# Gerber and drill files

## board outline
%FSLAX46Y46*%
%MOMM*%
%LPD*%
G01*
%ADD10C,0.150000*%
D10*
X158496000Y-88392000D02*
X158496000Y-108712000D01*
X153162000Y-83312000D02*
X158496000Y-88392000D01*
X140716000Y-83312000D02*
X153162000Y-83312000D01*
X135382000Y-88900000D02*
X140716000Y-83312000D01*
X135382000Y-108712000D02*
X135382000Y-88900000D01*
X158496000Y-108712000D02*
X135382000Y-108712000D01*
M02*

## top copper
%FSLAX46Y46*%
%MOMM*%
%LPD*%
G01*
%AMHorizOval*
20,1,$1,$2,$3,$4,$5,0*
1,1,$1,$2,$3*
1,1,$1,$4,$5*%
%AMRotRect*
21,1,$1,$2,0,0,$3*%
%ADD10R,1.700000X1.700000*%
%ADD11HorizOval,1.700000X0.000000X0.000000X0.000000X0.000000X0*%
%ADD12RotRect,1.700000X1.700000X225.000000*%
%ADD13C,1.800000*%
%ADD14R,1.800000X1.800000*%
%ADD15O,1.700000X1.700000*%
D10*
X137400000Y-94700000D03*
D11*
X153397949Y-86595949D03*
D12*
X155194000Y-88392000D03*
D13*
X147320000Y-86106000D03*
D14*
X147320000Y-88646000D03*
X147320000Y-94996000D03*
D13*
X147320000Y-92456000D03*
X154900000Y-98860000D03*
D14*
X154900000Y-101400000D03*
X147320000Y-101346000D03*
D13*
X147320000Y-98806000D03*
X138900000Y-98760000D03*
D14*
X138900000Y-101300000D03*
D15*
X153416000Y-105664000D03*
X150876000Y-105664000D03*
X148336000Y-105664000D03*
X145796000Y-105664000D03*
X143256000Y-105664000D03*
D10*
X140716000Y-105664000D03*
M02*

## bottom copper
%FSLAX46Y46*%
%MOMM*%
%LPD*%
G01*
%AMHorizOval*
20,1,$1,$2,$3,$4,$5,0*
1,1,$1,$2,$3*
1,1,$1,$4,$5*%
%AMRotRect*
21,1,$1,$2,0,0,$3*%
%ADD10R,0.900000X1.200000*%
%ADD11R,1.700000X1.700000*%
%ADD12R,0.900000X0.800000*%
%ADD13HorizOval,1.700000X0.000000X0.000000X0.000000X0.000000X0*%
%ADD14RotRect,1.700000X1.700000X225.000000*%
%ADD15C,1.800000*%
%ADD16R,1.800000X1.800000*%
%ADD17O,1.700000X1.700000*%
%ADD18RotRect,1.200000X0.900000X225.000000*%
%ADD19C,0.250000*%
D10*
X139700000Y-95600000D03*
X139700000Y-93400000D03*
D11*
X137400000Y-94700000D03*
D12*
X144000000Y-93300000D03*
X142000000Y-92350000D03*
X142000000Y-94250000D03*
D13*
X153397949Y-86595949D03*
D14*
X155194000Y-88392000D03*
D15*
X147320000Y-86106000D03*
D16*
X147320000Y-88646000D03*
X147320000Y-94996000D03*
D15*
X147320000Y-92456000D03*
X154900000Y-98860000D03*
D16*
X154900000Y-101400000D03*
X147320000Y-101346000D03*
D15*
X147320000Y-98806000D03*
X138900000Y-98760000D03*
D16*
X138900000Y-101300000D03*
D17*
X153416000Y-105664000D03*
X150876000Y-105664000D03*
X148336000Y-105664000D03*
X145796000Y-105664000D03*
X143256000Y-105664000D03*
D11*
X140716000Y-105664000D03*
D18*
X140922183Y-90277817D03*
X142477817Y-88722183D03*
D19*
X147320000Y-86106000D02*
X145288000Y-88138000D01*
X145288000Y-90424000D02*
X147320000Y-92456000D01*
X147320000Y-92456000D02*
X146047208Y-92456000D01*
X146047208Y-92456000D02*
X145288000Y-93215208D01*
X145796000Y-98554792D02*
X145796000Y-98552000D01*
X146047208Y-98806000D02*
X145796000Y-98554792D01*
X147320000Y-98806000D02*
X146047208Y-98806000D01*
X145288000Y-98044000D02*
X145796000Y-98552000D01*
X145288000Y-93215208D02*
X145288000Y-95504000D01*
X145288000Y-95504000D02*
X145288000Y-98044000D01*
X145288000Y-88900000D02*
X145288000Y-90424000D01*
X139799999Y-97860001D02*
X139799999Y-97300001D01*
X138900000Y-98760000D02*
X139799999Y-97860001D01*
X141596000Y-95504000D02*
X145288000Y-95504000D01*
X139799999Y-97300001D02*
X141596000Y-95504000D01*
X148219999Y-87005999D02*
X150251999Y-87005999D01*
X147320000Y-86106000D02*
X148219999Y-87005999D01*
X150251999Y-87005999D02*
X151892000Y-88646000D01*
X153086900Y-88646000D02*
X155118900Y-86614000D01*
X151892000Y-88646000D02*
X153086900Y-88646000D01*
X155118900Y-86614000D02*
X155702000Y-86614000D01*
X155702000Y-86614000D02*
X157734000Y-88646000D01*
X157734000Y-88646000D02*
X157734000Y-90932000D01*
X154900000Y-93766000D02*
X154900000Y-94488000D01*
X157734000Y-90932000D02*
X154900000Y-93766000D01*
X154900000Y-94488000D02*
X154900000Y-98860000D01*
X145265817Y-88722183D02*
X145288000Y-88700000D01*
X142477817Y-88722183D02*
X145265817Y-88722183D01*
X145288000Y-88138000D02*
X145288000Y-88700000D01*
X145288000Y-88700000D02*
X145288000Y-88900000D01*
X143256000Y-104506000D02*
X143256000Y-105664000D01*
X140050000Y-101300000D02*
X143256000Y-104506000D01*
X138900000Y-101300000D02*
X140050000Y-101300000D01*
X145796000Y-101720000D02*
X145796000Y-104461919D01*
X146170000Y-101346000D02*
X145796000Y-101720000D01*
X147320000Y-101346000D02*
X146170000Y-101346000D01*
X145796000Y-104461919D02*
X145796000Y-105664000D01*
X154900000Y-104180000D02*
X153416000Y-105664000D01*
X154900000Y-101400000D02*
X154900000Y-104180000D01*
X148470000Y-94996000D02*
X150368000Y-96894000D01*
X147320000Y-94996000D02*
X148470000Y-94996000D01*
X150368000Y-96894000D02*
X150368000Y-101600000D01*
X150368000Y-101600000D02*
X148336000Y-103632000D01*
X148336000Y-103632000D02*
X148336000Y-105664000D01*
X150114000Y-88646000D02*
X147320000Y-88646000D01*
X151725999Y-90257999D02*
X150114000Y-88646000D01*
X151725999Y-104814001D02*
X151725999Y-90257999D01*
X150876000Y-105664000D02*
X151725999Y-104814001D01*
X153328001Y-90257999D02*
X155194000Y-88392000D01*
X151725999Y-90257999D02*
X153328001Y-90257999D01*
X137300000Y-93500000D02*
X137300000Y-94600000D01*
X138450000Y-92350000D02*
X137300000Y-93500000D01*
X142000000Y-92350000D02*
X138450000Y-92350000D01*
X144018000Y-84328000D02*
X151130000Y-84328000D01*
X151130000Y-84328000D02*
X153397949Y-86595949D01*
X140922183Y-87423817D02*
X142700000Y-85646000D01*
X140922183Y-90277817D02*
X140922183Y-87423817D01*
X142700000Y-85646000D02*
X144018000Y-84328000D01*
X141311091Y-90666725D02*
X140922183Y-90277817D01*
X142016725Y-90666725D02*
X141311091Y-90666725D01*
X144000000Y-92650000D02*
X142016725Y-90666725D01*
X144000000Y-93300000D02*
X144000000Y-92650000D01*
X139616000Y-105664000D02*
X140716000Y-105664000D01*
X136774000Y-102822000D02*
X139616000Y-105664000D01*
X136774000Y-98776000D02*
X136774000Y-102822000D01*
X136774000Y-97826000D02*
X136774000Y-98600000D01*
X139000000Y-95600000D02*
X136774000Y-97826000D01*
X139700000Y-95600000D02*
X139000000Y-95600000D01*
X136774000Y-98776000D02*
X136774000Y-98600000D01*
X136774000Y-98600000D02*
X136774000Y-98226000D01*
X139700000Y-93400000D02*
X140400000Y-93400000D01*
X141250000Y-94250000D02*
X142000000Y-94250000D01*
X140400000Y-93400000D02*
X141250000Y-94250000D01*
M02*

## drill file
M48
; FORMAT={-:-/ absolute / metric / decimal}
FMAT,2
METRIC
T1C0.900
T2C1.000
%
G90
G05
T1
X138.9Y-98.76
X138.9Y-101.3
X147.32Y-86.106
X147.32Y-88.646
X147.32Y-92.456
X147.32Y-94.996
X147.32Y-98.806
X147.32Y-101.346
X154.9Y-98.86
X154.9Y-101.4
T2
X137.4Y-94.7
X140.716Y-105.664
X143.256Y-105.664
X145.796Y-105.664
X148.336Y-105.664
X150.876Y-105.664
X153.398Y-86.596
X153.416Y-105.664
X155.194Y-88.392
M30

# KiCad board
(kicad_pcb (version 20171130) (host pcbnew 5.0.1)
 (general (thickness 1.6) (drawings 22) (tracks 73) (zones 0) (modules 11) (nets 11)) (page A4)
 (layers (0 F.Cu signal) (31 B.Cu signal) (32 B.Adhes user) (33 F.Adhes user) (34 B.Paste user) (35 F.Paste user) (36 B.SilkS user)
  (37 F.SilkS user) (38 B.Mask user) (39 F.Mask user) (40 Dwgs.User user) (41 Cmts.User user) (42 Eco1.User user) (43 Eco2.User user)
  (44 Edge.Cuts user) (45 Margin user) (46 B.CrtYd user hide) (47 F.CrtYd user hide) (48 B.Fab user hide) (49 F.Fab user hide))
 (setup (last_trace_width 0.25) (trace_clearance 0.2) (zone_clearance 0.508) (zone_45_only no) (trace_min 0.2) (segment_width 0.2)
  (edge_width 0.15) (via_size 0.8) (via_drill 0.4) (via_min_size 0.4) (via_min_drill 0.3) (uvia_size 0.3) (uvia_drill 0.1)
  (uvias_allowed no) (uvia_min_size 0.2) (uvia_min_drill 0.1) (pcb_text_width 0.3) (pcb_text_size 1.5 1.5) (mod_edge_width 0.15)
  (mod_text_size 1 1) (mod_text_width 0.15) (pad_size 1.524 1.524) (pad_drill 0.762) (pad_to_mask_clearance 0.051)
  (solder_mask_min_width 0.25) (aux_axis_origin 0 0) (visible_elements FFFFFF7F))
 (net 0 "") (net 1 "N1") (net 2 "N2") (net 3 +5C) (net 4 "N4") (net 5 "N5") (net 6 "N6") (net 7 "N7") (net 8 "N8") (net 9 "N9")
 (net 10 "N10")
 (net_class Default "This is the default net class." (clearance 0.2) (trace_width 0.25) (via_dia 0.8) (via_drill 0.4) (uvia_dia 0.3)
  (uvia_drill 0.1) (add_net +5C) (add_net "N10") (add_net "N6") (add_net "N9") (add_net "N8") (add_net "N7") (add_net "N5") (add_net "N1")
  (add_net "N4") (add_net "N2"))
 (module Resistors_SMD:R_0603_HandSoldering (layer B.Cu) (at 139.7 94.5 270)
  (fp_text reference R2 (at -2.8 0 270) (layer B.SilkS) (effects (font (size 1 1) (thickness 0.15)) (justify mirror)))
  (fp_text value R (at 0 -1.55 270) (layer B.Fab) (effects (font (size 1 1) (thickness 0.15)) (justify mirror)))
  (pad 2 smd rect (at 1.1 0 270) (size 1.2 0.9) (layers B.Cu B.Paste B.Mask) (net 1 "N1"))
  (pad 1 smd rect (at -1.1 0 270) (size 1.2 0.9) (layers B.Cu B.Paste B.Mask) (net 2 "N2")))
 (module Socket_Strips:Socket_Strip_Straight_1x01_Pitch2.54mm (layer F.Cu) (at 137.4 94.7)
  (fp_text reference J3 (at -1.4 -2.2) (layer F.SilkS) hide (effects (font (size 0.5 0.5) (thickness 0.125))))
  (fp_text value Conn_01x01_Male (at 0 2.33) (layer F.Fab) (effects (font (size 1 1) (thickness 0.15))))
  (pad 1 thru_hole rect (at 0 0) (size 1.7 1.7) (drill 1) (layers *.Cu *.Mask) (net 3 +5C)))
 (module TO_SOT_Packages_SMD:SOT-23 (layer B.Cu) (at 143 93.3)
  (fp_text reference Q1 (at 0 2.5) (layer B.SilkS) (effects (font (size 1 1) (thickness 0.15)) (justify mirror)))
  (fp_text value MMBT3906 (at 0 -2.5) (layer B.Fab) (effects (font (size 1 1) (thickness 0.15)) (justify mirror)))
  (pad 3 smd rect (at 1 0) (size 0.9 0.8) (layers B.Cu B.Paste B.Mask) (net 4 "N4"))
  (pad 2 smd rect (at -1 -0.95) (size 0.9 0.8) (layers B.Cu B.Paste B.Mask) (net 3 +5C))
  (pad 1 smd rect (at -1 0.95) (size 0.9 0.8) (layers B.Cu B.Paste B.Mask) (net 2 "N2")))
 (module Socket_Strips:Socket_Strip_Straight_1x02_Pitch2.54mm (layer F.Cu) (at 155.194 88.392 225)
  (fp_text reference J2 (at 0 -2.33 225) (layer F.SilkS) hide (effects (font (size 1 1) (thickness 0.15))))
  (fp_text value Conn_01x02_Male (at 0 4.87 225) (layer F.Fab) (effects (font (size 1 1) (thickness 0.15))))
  (pad 2 thru_hole oval (at 0 2.54 225) (size 1.7 1.7) (drill 1) (layers *.Cu *.Mask) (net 4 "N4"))
  (pad 1 thru_hole rect (at 0 0 225) (size 1.7 1.7) (drill 1) (layers *.Cu *.Mask) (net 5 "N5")))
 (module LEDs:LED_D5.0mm (layer F.Cu) (at 147.32 88.646 90)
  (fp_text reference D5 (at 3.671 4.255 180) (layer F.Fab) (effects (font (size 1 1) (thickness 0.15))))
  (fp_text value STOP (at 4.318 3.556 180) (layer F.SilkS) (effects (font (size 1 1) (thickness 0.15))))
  (pad 2 thru_hole circle (at 2.54 0 90) (size 1.8 1.8) (drill 0.9) (layers *.Cu *.Mask) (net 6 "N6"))
  (pad 1 thru_hole rect (at 0 0 90) (size 1.8 1.8) (drill 0.9) (layers *.Cu *.Mask) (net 5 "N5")))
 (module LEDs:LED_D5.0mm (layer F.Cu) (at 147.32 94.996 90)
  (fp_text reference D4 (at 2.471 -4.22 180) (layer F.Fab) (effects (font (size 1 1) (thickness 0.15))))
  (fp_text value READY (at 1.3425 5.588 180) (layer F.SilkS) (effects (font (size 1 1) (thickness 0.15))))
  (pad 1 thru_hole rect (at 0 0 90) (size 1.8 1.8) (drill 0.9) (layers *.Cu *.Mask) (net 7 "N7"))
  (pad 2 thru_hole circle (at 2.54 0 90) (size 1.8 1.8) (drill 0.9) (layers *.Cu *.Mask) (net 6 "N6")))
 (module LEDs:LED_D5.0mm (layer F.Cu) (at 154.9 101.4 90)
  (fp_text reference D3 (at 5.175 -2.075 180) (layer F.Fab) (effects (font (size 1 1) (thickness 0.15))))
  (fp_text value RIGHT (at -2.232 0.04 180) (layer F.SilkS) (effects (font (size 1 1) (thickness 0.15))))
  (pad 2 thru_hole circle (at 2.54 0 90) (size 1.8 1.8) (drill 0.9) (layers *.Cu *.Mask) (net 6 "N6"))
  (pad 1 thru_hole rect (at 0 0 90) (size 1.8 1.8) (drill 0.9) (layers *.Cu *.Mask) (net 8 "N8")))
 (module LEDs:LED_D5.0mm (layer F.Cu) (at 147.32 101.346 90)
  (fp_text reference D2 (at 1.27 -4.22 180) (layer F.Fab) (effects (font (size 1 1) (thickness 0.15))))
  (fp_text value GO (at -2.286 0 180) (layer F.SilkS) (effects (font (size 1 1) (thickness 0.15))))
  (pad 1 thru_hole rect (at 0 0 90) (size 1.8 1.8) (drill 0.9) (layers *.Cu *.Mask) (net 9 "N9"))
  (pad 2 thru_hole circle (at 2.54 0 90) (size 1.8 1.8) (drill 0.9) (layers *.Cu *.Mask) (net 6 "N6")))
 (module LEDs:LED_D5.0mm (layer F.Cu) (at 138.9 101.3 90)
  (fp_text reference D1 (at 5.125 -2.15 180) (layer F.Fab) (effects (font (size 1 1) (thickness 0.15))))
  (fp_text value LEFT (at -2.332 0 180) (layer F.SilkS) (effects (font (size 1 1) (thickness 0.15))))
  (pad 2 thru_hole circle (at 2.54 0 90) (size 1.8 1.8) (drill 0.9) (layers *.Cu *.Mask) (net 6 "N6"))
  (pad 1 thru_hole rect (at 0 0 90) (size 1.8 1.8) (drill 0.9) (layers *.Cu *.Mask) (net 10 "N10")))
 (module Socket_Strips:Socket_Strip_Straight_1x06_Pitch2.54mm (layer F.Cu) (at 140.716 105.664 90)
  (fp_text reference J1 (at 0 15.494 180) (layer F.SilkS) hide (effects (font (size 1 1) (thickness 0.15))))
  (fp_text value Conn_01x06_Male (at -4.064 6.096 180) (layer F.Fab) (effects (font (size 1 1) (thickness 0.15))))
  (pad 6 thru_hole oval (at 0 12.7 90) (size 1.7 1.7) (drill 1) (layers *.Cu *.Mask) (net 8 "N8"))
  (pad 5 thru_hole oval (at 0 10.16 90) (size 1.7 1.7) (drill 1) (layers *.Cu *.Mask) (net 5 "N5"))
  (pad 4 thru_hole oval (at 0 7.62 90) (size 1.7 1.7) (drill 1) (layers *.Cu *.Mask) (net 7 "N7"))
  (pad 3 thru_hole oval (at 0 5.08 90) (size 1.7 1.7) (drill 1) (layers *.Cu *.Mask) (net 9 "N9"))
  (pad 2 thru_hole oval (at 0 2.54 90) (size 1.7 1.7) (drill 1) (layers *.Cu *.Mask) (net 10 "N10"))
  (pad 1 thru_hole rect (at 0 0 90) (size 1.7 1.7) (drill 1) (layers *.Cu *.Mask) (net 1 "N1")))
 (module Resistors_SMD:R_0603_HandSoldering (layer B.Cu) (at 141.7 89.5 225)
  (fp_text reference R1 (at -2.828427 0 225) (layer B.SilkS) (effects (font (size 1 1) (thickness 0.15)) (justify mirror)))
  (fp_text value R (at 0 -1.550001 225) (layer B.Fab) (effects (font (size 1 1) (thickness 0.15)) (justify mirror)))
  (pad 2 smd rect (at 1.099999 0 225) (size 1.2 0.9) (layers B.Cu B.Paste B.Mask) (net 4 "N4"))
  (pad 1 smd rect (at -1.099999 0 225) (size 1.2 0.9) (layers B.Cu B.Paste B.Mask) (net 6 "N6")))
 (gr_line (start 158.496 88.392) (end 158.496 108.712) (layer Edge.Cuts) (width 0.15))
 (gr_line (start 153.162 83.312) (end 158.496 88.392) (layer Edge.Cuts) (width 0.15))
 (gr_line (start 140.716 83.312) (end 153.162 83.312) (layer Edge.Cuts) (width 0.15))
 (gr_line (start 135.382 88.9) (end 140.716 83.312) (layer Edge.Cuts) (width 0.15))
 (gr_line (start 135.382 108.712) (end 135.382 88.9) (layer Edge.Cuts) (width 0.15))
 (gr_line (start 158.496 108.712) (end 135.382 108.712) (layer Edge.Cuts) (width 0.15))
 (segment (start 147.32 86.106) (end 145.288 88.138) (width 0.25) (layer B.Cu) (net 6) (status 10))
 (segment (start 145.288 90.424) (end 147.32 92.456) (width 0.25) (layer B.Cu) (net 6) (status 20))
 (segment (start 147.32 92.456) (end 146.047208 92.456) (width 0.25) (layer B.Cu) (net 6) (status 10))
 (segment (start 146.047208 92.456) (end 145.288 93.215208) (width 0.25) (layer B.Cu) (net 6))
 (segment (start 145.796 98.554792) (end 145.796 98.552) (width 0.25) (layer B.Cu) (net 6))
 (segment (start 146.047208 98.806) (end 145.796 98.554792) (width 0.25) (layer B.Cu) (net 6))
 (segment (start 147.32 98.806) (end 146.047208 98.806) (width 0.25) (layer B.Cu) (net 6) (status 10))
 (segment (start 145.288 98.044) (end 145.796 98.552) (width 0.25) (layer B.Cu) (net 6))
 (segment (start 145.288 93.215208) (end 145.288 95.504) (width 0.25) (layer B.Cu) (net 6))
 (segment (start 145.288 95.504) (end 145.288 98.044) (width 0.25) (layer B.Cu) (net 6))
 (segment (start 145.288 88.9) (end 145.288 90.424) (width 0.25) (layer B.Cu) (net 6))
 (segment (start 139.799999 97.860001) (end 139.799999 97.300001) (width 0.25) (layer B.Cu) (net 6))
 (segment (start 138.9 98.76) (end 139.799999 97.860001) (width 0.25) (layer B.Cu) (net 6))
 (segment (start 141.596 95.504) (end 145.288 95.504) (width 0.25) (layer B.Cu) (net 6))
 (segment (start 139.799999 97.300001) (end 141.596 95.504) (width 0.25) (layer B.Cu) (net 6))
 (segment (start 148.219999 87.005999) (end 150.251999 87.005999) (width 0.25) (layer B.Cu) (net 6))
 (segment (start 147.32 86.106) (end 148.219999 87.005999) (width 0.25) (layer B.Cu) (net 6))
 (segment (start 150.251999 87.005999) (end 151.892 88.646) (width 0.25) (layer B.Cu) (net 6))
 (segment (start 153.0869 88.646) (end 155.1189 86.614) (width 0.25) (layer B.Cu) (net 6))
 (segment (start 151.892 88.646) (end 153.0869 88.646) (width 0.25) (layer B.Cu) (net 6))
 (segment (start 155.1189 86.614) (end 155.702 86.614) (width 0.25) (layer B.Cu) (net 6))
 (segment (start 155.702 86.614) (end 157.734 88.646) (width 0.25) (layer B.Cu) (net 6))
 (segment (start 157.734 88.646) (end 157.734 90.932) (width 0.25) (layer B.Cu) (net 6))
 (segment (start 154.9 93.766) (end 154.9 94.488) (width 0.25) (layer B.Cu) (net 6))
 (segment (start 157.734 90.932) (end 154.9 93.766) (width 0.25) (layer B.Cu) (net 6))
 (segment (start 154.9 94.488) (end 154.9 98.86) (width 0.25) (layer B.Cu) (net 6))
 (segment (start 145.265817 88.722183) (end 145.288 88.7) (width 0.25) (layer B.Cu) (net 6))
 (segment (start 142.477817 88.722183) (end 145.265817 88.722183) (width 0.25) (layer B.Cu) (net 6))
 (segment (start 145.288 88.138) (end 145.288 88.7) (width 0.25) (layer B.Cu) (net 6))
 (segment (start 145.288 88.7) (end 145.288 88.9) (width 0.25) (layer B.Cu) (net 6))
 (segment (start 143.256 104.506) (end 143.256 105.664) (width 0.25) (layer B.Cu) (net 10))
 (segment (start 140.05 101.3) (end 143.256 104.506) (width 0.25) (layer B.Cu) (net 10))
 (segment (start 138.9 101.3) (end 140.05 101.3) (width 0.25) (layer B.Cu) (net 10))
 (segment (start 145.796 101.72) (end 145.796 104.461919) (width 0.25) (layer B.Cu) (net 9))
 (segment (start 146.17 101.346) (end 145.796 101.72) (width 0.25) (layer B.Cu) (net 9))
 (segment (start 147.32 101.346) (end 146.17 101.346) (width 0.25) (layer B.Cu) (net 9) (status 10))
 (segment (start 145.796 104.461919) (end 145.796 105.664) (width 0.25) (layer B.Cu) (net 9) (status 20))
 (segment (start 154.9 104.18) (end 153.416 105.664) (width 0.25) (layer B.Cu) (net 8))
 (segment (start 154.9 101.4) (end 154.9 104.18) (width 0.25) (layer B.Cu) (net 8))
 (segment (start 148.47 94.996) (end 150.368 96.894) (width 0.25) (layer B.Cu) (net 7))
 (segment (start 147.32 94.996) (end 148.47 94.996) (width 0.25) (layer B.Cu) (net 7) (status 10))
 (segment (start 150.368 96.894) (end 150.368 101.6) (width 0.25) (layer B.Cu) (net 7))
 (segment (start 150.368 101.6) (end 148.336 103.632) (width 0.25) (layer B.Cu) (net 7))
 (segment (start 148.336 103.632) (end 148.336 105.664) (width 0.25) (layer B.Cu) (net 7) (status 20))
 (segment (start 150.114 88.646) (end 147.32 88.646) (width 0.25) (layer B.Cu) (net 5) (status 20))
 (segment (start 151.725999 90.257999) (end 150.114 88.646) (width 0.25) (layer B.Cu) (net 5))
 (segment (start 151.725999 104.814001) (end 151.725999 90.257999) (width 0.25) (layer B.Cu) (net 5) (status 10))
 (segment (start 150.876 105.664) (end 151.725999 104.814001) (width 0.25) (layer B.Cu) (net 5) (status 30))
 (segment (start 153.328001 90.257999) (end 155.194 88.392) (width 0.25) (layer B.Cu) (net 5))
 (segment (start 151.725999 90.257999) (end 153.328001 90.257999) (width 0.25) (layer B.Cu) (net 5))
 (segment (start 137.3 93.5) (end 137.3 94.6) (width 0.25) (layer B.Cu) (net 3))
 (segment (start 138.45 92.35) (end 137.3 93.5) (width 0.25) (layer B.Cu) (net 3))
 (segment (start 142 92.35) (end 138.45 92.35) (width 0.25) (layer B.Cu) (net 3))
 (segment (start 144.018 84.328) (end 151.13 84.328) (width 0.25) (layer B.Cu) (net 4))
 (segment (start 151.13 84.328) (end 153.397949 86.595949) (width 0.25) (layer B.Cu) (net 4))
 (segment (start 140.922183 87.423817) (end 142.7 85.646) (width 0.25) (layer B.Cu) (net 4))
 (segment (start 140.922183 90.277817) (end 140.922183 87.423817) (width 0.25) (layer B.Cu) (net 4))
 (segment (start 142.7 85.646) (end 144.018 84.328) (width 0.25) (layer B.Cu) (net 4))
 (segment (start 141.311091 90.666725) (end 140.922183 90.277817) (width 0.25) (layer B.Cu) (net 4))
 (segment (start 142.016725 90.666725) (end 141.311091 90.666725) (width 0.25) (layer B.Cu) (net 4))
 (segment (start 144 92.65) (end 142.016725 90.666725) (width 0.25) (layer B.Cu) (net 4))
 (segment (start 144 93.3) (end 144 92.65) (width 0.25) (layer B.Cu) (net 4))
 (segment (start 139.616 105.664) (end 140.716 105.664) (width 0.25) (layer B.Cu) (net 1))
 (segment (start 136.774 102.822) (end 139.616 105.664) (width 0.25) (layer B.Cu) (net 1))
 (segment (start 136.774 98.776) (end 136.774 102.822) (width 0.25) (layer B.Cu) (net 1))
 (segment (start 136.774 97.826) (end 136.774 98.6) (width 0.25) (layer B.Cu) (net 1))
 (segment (start 139 95.6) (end 136.774 97.826) (width 0.25) (layer B.Cu) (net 1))
 (segment (start 139.7 95.6) (end 139 95.6) (width 0.25) (layer B.Cu) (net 1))
 (segment (start 136.774 98.776) (end 136.774 98.6) (width 0.25) (layer B.Cu) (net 1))
 (segment (start 136.774 98.6) (end 136.774 98.226) (width 0.25) (layer B.Cu) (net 1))
 (segment (start 139.7 93.4) (end 140.4 93.4) (width 0.25) (layer B.Cu) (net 2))
 (segment (start 141.25 94.25) (end 142 94.25) (width 0.25) (layer B.Cu) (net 2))
 (segment (start 140.4 93.4) (end 141.25 94.25) (width 0.25) (layer B.Cu) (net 2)))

